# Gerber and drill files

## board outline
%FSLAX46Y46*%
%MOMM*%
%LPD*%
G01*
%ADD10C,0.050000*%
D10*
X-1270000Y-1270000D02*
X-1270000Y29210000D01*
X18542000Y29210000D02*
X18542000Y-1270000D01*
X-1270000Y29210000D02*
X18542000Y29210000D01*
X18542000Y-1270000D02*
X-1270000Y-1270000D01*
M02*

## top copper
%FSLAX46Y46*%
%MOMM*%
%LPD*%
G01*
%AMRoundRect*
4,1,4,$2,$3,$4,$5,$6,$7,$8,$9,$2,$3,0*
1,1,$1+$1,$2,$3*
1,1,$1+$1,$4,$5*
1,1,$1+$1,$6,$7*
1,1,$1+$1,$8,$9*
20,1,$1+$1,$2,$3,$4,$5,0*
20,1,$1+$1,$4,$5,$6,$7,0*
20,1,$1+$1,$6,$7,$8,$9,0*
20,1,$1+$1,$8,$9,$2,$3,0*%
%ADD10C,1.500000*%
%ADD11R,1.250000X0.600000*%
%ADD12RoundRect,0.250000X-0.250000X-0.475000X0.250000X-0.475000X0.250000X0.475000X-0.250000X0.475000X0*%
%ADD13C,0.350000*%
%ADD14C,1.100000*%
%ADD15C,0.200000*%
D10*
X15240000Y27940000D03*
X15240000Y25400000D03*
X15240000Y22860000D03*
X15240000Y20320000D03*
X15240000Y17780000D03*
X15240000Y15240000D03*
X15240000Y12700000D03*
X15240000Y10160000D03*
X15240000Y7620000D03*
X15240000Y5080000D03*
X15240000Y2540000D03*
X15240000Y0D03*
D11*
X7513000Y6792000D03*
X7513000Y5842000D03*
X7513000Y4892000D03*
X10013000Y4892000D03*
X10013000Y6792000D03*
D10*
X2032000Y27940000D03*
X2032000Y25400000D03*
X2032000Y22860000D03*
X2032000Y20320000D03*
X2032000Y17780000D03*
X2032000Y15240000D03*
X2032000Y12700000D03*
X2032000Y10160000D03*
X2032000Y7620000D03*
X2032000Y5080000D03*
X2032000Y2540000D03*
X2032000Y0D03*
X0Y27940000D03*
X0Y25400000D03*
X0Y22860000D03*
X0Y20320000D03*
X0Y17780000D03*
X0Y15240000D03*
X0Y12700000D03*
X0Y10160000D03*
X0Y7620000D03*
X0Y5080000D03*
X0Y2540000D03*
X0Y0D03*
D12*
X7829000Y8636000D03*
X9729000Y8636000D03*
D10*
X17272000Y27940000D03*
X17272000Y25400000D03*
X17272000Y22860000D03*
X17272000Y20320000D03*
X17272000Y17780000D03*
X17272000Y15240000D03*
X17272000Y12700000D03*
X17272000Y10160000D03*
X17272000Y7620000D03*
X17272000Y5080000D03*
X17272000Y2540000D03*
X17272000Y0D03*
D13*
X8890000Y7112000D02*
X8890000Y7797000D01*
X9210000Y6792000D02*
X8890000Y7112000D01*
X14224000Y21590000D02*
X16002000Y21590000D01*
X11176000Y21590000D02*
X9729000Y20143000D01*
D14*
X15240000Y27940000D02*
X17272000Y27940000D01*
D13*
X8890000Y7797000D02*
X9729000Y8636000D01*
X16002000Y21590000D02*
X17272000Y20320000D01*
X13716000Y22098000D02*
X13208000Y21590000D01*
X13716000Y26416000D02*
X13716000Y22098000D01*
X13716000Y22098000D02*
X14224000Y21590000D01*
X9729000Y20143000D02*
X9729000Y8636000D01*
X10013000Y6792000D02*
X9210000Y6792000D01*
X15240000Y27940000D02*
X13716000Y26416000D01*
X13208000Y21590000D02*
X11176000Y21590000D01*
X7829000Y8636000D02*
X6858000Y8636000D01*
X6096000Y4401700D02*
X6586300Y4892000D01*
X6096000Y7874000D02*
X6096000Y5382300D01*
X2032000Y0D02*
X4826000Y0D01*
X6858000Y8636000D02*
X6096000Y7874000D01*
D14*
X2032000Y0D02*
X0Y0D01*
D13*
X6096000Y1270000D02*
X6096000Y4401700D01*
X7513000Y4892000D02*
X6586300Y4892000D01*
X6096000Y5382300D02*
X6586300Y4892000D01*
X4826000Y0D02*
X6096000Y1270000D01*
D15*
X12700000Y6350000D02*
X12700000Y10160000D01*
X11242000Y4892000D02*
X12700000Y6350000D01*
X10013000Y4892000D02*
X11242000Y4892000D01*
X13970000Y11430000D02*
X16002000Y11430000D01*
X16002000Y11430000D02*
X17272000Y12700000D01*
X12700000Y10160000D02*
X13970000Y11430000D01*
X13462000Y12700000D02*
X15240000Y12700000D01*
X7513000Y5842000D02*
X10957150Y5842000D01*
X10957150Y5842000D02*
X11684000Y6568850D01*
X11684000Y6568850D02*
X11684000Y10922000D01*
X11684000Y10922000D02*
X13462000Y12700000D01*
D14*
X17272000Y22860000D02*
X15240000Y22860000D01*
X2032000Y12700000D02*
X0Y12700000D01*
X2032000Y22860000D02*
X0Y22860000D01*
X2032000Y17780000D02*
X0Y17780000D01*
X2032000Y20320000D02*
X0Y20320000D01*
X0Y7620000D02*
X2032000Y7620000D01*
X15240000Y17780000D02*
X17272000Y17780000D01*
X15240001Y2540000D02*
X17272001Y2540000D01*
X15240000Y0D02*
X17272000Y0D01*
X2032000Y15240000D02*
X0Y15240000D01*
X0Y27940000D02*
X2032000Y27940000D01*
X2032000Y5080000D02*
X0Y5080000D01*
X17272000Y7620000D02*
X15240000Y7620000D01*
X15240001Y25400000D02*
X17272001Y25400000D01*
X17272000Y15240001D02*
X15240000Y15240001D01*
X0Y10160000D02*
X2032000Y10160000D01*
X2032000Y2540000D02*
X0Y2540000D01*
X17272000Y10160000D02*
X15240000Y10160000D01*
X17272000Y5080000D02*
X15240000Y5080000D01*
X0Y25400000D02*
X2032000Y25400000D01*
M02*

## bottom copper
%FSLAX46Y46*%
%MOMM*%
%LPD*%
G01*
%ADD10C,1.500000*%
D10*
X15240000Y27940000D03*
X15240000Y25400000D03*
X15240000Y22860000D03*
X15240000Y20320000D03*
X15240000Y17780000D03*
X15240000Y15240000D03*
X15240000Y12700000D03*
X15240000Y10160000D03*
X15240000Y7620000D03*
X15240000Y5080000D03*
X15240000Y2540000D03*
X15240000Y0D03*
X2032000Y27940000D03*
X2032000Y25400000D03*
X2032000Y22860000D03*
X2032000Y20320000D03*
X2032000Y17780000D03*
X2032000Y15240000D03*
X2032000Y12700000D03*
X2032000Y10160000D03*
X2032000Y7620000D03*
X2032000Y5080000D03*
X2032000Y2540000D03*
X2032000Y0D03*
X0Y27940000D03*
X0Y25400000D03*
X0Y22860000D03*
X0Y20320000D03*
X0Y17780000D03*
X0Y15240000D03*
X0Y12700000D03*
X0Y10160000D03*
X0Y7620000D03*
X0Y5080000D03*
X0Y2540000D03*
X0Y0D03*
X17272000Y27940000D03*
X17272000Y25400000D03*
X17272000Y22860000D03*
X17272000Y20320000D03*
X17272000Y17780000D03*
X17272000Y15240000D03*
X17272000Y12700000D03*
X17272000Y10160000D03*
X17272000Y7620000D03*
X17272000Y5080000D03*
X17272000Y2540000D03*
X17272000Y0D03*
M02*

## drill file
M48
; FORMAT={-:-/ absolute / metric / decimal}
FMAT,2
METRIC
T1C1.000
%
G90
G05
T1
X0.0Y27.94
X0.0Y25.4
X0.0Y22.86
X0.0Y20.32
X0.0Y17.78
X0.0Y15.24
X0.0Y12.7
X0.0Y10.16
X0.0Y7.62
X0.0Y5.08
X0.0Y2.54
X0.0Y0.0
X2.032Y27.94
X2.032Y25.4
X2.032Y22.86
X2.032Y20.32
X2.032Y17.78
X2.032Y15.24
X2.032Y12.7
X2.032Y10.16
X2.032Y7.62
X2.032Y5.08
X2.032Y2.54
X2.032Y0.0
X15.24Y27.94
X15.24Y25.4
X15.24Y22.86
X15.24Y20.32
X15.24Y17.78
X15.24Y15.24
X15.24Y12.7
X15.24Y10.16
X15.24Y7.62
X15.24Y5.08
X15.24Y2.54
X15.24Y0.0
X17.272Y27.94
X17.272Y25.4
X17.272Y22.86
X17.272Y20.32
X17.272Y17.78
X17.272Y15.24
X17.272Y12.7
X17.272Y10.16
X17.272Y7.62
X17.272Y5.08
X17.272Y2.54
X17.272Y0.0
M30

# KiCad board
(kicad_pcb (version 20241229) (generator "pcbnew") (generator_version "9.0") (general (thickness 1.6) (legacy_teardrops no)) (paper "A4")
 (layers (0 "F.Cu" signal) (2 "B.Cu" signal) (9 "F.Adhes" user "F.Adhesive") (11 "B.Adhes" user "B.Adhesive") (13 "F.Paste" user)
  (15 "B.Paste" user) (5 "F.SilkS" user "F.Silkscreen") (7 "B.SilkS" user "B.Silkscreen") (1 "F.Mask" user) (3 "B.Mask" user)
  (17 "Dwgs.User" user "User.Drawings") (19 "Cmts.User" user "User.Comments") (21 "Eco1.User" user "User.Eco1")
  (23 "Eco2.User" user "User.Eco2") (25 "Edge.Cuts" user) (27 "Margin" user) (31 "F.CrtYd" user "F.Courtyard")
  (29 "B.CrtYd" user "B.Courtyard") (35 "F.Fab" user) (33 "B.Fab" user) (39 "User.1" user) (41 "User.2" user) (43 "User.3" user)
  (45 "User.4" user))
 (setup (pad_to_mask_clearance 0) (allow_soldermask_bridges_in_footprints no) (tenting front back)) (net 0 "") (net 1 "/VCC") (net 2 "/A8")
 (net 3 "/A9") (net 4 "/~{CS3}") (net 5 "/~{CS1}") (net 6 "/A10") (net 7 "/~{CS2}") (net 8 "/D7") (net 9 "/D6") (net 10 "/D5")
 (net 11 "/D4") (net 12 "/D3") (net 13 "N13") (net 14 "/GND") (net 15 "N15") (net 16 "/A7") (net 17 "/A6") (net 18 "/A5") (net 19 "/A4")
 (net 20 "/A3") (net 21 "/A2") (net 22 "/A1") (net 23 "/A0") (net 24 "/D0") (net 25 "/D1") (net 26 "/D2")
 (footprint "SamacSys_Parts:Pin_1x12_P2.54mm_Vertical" (layer "F.Cu") (at 15.24 -27.94)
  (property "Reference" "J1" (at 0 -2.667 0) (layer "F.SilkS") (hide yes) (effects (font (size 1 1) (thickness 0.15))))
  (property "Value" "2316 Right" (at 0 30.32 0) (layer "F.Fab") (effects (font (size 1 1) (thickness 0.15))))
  (pad "1" thru_hole circle (at 0 0) (size 1.5 1.5) (drill 1) (layers "*.Cu" "*.Mask") (remove_unused_layers no) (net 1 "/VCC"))
  (pad "2" thru_hole circle (at 0 2.54) (size 1.5 1.5) (drill 1) (layers "*.Cu" "*.Mask") (remove_unused_layers no) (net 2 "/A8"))
  (pad "3" thru_hole circle (at 0 5.08) (size 1.5 1.5) (drill 1) (layers "*.Cu" "*.Mask") (remove_unused_layers no) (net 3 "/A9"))
  (pad "4" thru_hole circle (at 0 7.62) (size 1.5 1.5) (drill 1) (layers "*.Cu" "*.Mask") (remove_unused_layers no) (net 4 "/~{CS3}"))
  (pad "5" thru_hole circle (at 0 10.16) (size 1.5 1.5) (drill 1) (layers "*.Cu" "*.Mask") (remove_unused_layers no) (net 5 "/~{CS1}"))
  (pad "6" thru_hole circle (at 0 12.7) (size 1.5 1.5) (drill 1) (layers "*.Cu" "*.Mask") (remove_unused_layers no) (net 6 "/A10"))
  (pad "7" thru_hole circle (at 0 15.24) (size 1.5 1.5) (drill 1) (layers "*.Cu" "*.Mask") (remove_unused_layers no) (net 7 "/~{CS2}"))
  (pad "8" thru_hole circle (at 0 17.78) (size 1.5 1.5) (drill 1) (layers "*.Cu" "*.Mask") (remove_unused_layers no) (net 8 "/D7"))
  (pad "9" thru_hole circle (at 0 20.32) (size 1.5 1.5) (drill 1) (layers "*.Cu" "*.Mask") (remove_unused_layers no) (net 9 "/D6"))
  (pad "10" thru_hole circle (at 0 22.86) (size 1.5 1.5) (drill 1) (layers "*.Cu" "*.Mask") (remove_unused_layers no) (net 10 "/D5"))
  (pad "11" thru_hole circle (at 0 25.4) (size 1.5 1.5) (drill 1) (layers "*.Cu" "*.Mask") (remove_unused_layers no) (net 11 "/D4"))
  (pad "12" thru_hole circle (at 0 27.94) (size 1.5 1.5) (drill 1) (layers "*.Cu" "*.Mask") (remove_unused_layers no) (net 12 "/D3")))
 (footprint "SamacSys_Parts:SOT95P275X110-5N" (layer "F.Cu") (at 8.763 -5.842)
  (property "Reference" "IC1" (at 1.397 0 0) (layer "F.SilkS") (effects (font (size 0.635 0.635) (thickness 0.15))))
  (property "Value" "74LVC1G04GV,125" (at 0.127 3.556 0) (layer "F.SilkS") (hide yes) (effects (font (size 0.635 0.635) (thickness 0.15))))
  (pad "1" smd rect (at -1.25 -0.95 90) (size 0.6 1.25) (layers "F.Cu" "F.Mask" "F.Paste") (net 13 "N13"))
  (pad "2" smd rect (at -1.25 0 90) (size 0.6 1.25) (layers "F.Cu" "F.Mask" "F.Paste") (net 7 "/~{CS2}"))
  (pad "3" smd rect (at -1.25 0.95 90) (size 0.6 1.25) (layers "F.Cu" "F.Mask" "F.Paste") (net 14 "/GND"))
  (pad "4" smd rect (at 1.25 0.95 90) (size 0.6 1.25) (layers "F.Cu" "F.Mask" "F.Paste") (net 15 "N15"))
  (pad "5" smd rect (at 1.25 -0.95 90) (size 0.6 1.25) (layers "F.Cu" "F.Mask" "F.Paste") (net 1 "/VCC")))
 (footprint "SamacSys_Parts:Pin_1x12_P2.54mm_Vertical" (layer "F.Cu") (at 2.032 -27.94)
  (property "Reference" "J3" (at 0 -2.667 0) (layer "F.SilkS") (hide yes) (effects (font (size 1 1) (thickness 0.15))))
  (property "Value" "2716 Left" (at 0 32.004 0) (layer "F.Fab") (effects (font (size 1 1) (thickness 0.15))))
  (pad "1" thru_hole circle (at 0 0) (size 1.5 1.5) (drill 1) (layers "*.Cu" "*.Mask") (remove_unused_layers no) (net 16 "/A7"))
  (pad "2" thru_hole circle (at 0 2.54) (size 1.5 1.5) (drill 1) (layers "*.Cu" "*.Mask") (remove_unused_layers no) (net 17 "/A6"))
  (pad "3" thru_hole circle (at 0 5.08) (size 1.5 1.5) (drill 1) (layers "*.Cu" "*.Mask") (remove_unused_layers no) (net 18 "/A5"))
  (pad "4" thru_hole circle (at 0 7.62) (size 1.5 1.5) (drill 1) (layers "*.Cu" "*.Mask") (remove_unused_layers no) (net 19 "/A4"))
  (pad "5" thru_hole circle (at 0 10.16) (size 1.5 1.5) (drill 1) (layers "*.Cu" "*.Mask") (remove_unused_layers no) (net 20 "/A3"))
  (pad "6" thru_hole circle (at 0 12.7) (size 1.5 1.5) (drill 1) (layers "*.Cu" "*.Mask") (remove_unused_layers no) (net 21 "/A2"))
  (pad "7" thru_hole circle (at 0 15.24) (size 1.5 1.5) (drill 1) (layers "*.Cu" "*.Mask") (remove_unused_layers no) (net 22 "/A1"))
  (pad "8" thru_hole circle (at 0 17.78) (size 1.5 1.5) (drill 1) (layers "*.Cu" "*.Mask") (remove_unused_layers no) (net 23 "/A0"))
  (pad "9" thru_hole circle (at 0 20.32) (size 1.5 1.5) (drill 1) (layers "*.Cu" "*.Mask") (remove_unused_layers no) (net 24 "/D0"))
  (pad "10" thru_hole circle (at 0 22.86) (size 1.5 1.5) (drill 1) (layers "*.Cu" "*.Mask") (remove_unused_layers no) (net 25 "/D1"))
  (pad "11" thru_hole circle (at 0 25.4) (size 1.5 1.5) (drill 1) (layers "*.Cu" "*.Mask") (remove_unused_layers no) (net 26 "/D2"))
  (pad "12" thru_hole circle (at 0 27.94) (size 1.5 1.5) (drill 1) (layers "*.Cu" "*.Mask") (remove_unused_layers no) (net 14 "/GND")))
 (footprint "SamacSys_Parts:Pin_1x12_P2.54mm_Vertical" (layer "F.Cu") (at 0 -27.94)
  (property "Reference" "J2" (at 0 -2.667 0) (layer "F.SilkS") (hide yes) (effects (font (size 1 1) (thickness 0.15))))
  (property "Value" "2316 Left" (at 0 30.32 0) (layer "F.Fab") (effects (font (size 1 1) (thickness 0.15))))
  (pad "1" thru_hole circle (at 0 0) (size 1.5 1.5) (drill 1) (layers "*.Cu" "*.Mask") (remove_unused_layers no) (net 16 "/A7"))
  (pad "2" thru_hole circle (at 0 2.54) (size 1.5 1.5) (drill 1) (layers "*.Cu" "*.Mask") (remove_unused_layers no) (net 17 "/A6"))
  (pad "3" thru_hole circle (at 0 5.08) (size 1.5 1.5) (drill 1) (layers "*.Cu" "*.Mask") (remove_unused_layers no) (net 18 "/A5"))
  (pad "4" thru_hole circle (at 0 7.62) (size 1.5 1.5) (drill 1) (layers "*.Cu" "*.Mask") (remove_unused_layers no) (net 19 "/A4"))
  (pad "5" thru_hole circle (at 0 10.16) (size 1.5 1.5) (drill 1) (layers "*.Cu" "*.Mask") (remove_unused_layers no) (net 20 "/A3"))
  (pad "6" thru_hole circle (at 0 12.7) (size 1.5 1.5) (drill 1) (layers "*.Cu" "*.Mask") (remove_unused_layers no) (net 21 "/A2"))
  (pad "7" thru_hole circle (at 0 15.24) (size 1.5 1.5) (drill 1) (layers "*.Cu" "*.Mask") (remove_unused_layers no) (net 22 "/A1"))
  (pad "8" thru_hole circle (at 0 17.78) (size 1.5 1.5) (drill 1) (layers "*.Cu" "*.Mask") (remove_unused_layers no) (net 23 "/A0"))
  (pad "9" thru_hole circle (at 0 20.32) (size 1.5 1.5) (drill 1) (layers "*.Cu" "*.Mask") (remove_unused_layers no) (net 24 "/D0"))
  (pad "10" thru_hole circle (at 0 22.86) (size 1.5 1.5) (drill 1) (layers "*.Cu" "*.Mask") (remove_unused_layers no) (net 25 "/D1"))
  (pad "11" thru_hole circle (at 0 25.4) (size 1.5 1.5) (drill 1) (layers "*.Cu" "*.Mask") (remove_unused_layers no) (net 26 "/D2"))
  (pad "12" thru_hole circle (at 0 27.94) (size 1.5 1.5) (drill 1) (layers "*.Cu" "*.Mask") (remove_unused_layers no) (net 14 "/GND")))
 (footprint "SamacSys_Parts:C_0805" (layer "F.Cu") (at 8.763 -8.636 -90)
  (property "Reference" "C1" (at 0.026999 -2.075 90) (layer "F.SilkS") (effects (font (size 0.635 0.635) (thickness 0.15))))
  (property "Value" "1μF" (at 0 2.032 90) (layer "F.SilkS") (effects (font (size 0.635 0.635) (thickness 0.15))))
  (pad "1" smd roundrect (at 0 0.934) (size 1 1.45) (layers "F.Cu" "F.Mask" "F.Paste") (roundrect_rratio 0.25) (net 14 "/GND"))
  (pad "2" smd roundrect (at 0 -0.966) (size 1 1.45) (layers "F.Cu" "F.Mask" "F.Paste") (roundrect_rratio 0.25) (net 1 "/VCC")))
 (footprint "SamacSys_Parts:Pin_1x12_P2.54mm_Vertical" (layer "F.Cu") (at 17.272 -27.94)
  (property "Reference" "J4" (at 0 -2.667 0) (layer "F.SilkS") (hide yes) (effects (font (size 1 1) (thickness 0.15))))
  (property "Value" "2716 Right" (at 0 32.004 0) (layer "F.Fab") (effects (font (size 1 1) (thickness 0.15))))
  (pad "1" thru_hole circle (at 0 0) (size 1.5 1.5) (drill 1) (layers "*.Cu" "*.Mask") (remove_unused_layers no) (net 1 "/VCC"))
  (pad "2" thru_hole circle (at 0 2.54) (size 1.5 1.5) (drill 1) (layers "*.Cu" "*.Mask") (remove_unused_layers no) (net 2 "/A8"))
  (pad "3" thru_hole circle (at 0 5.08) (size 1.5 1.5) (drill 1) (layers "*.Cu" "*.Mask") (remove_unused_layers no) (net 3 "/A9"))
  (pad "4" thru_hole circle (at 0 7.62) (size 1.5 1.5) (drill 1) (layers "*.Cu" "*.Mask") (remove_unused_layers no) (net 1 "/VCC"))
  (pad "5" thru_hole circle (at 0 10.16) (size 1.5 1.5) (drill 1) (layers "*.Cu" "*.Mask") (remove_unused_layers no) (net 5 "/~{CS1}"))
  (pad "6" thru_hole circle (at 0 12.7) (size 1.5 1.5) (drill 1) (layers "*.Cu" "*.Mask") (remove_unused_layers no) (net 6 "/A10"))
  (pad "7" thru_hole circle (at 0 15.24) (size 1.5 1.5) (drill 1) (layers "*.Cu" "*.Mask") (remove_unused_layers no) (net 15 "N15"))
  (pad "8" thru_hole circle (at 0 17.78) (size 1.5 1.5) (drill 1) (layers "*.Cu" "*.Mask") (remove_unused_layers no) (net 8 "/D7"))
  (pad "9" thru_hole circle (at 0 20.32) (size 1.5 1.5) (drill 1) (layers "*.Cu" "*.Mask") (remove_unused_layers no) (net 9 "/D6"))
  (pad "10" thru_hole circle (at 0 22.86) (size 1.5 1.5) (drill 1) (layers "*.Cu" "*.Mask") (remove_unused_layers no) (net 10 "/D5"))
  (pad "11" thru_hole circle (at 0 25.4) (size 1.5 1.5) (drill 1) (layers "*.Cu" "*.Mask") (remove_unused_layers no) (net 11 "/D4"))
  (pad "12" thru_hole circle (at 0 27.94) (size 1.5 1.5) (drill 1) (layers "*.Cu" "*.Mask") (remove_unused_layers no) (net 12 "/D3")))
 (gr_line (start -1.27 1.27) (end -1.27 -29.21) (stroke (width 0.05) (type default)) (layer "Edge.Cuts"))
 (gr_line (start 18.542 -29.21) (end 18.542 1.27) (stroke (width 0.05) (type default)) (layer "Edge.Cuts"))
 (gr_line (start -1.27 -29.21) (end 18.542 -29.21) (stroke (width 0.05) (type default)) (layer "Edge.Cuts"))
 (gr_line (start 18.542 1.27) (end -1.27 1.27) (stroke (width 0.05) (type default)) (layer "Edge.Cuts"))
 (segment (start 8.89 -7.112) (end 8.89 -7.797) (width 0.35) (layer "F.Cu") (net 1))
 (segment (start 9.21 -6.792) (end 8.89 -7.112) (width 0.35) (layer "F.Cu") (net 1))
 (segment (start 14.224 -21.59) (end 16.002 -21.59) (width 0.35) (layer "F.Cu") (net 1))
 (segment (start 11.176 -21.59) (end 9.729 -20.143) (width 0.35) (layer "F.Cu") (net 1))
 (segment (start 15.24 -27.94) (end 17.272 -27.94) (width 1.1) (layer "F.Cu") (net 1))
 (segment (start 8.89 -7.797) (end 9.729 -8.636) (width 0.35) (layer "F.Cu") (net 1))
 (segment (start 16.002 -21.59) (end 17.272 -20.32) (width 0.35) (layer "F.Cu") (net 1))
 (segment (start 13.716 -22.098) (end 13.208 -21.59) (width 0.35) (layer "F.Cu") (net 1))
 (segment (start 13.716 -26.416) (end 13.716 -22.098) (width 0.35) (layer "F.Cu") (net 1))
 (segment (start 13.716 -22.098) (end 14.224 -21.59) (width 0.35) (layer "F.Cu") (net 1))
 (segment (start 9.729 -20.143) (end 9.729 -8.636) (width 0.35) (layer "F.Cu") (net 1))
 (segment (start 10.013 -6.792) (end 9.21 -6.792) (width 0.35) (layer "F.Cu") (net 1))
 (segment (start 15.24 -27.94) (end 13.716 -26.416) (width 0.35) (layer "F.Cu") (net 1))
 (segment (start 13.208 -21.59) (end 11.176 -21.59) (width 0.35) (layer "F.Cu") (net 1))
 (segment (start 7.829 -8.636) (end 6.858 -8.636) (width 0.35) (layer "F.Cu") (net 14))
 (segment (start 6.096 -4.4017) (end 6.5863 -4.892) (width 0.35) (layer "F.Cu") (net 14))
 (segment (start 6.096 -7.874) (end 6.096 -5.3823) (width 0.35) (layer "F.Cu") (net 14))
 (segment (start 2.032 0) (end 4.826 0) (width 0.35) (layer "F.Cu") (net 14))
 (segment (start 6.858 -8.636) (end 6.096 -7.874) (width 0.35) (layer "F.Cu") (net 14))
 (segment (start 2.032 0) (end 0 0) (width 1.1) (layer "F.Cu") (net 14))
 (segment (start 6.096 -1.27) (end 6.096 -4.4017) (width 0.35) (layer "F.Cu") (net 14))
 (segment (start 7.513 -4.892) (end 6.5863 -4.892) (width 0.35) (layer "F.Cu") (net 14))
 (segment (start 6.096 -5.3823) (end 6.5863 -4.892) (width 0.35) (layer "F.Cu") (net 14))
 (segment (start 4.826 0) (end 6.096 -1.27) (width 0.35) (layer "F.Cu") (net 14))
 (segment (start 12.7 -6.35) (end 12.7 -10.16) (width 0.2) (layer "F.Cu") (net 15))
 (segment (start 11.242 -4.892) (end 12.7 -6.35) (width 0.2) (layer "F.Cu") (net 15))
 (segment (start 10.013 -4.892) (end 11.242 -4.892) (width 0.2) (layer "F.Cu") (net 15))
 (segment (start 13.97 -11.43) (end 16.002 -11.43) (width 0.2) (layer "F.Cu") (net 15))
 (segment (start 16.002 -11.43) (end 17.272 -12.7) (width 0.2) (layer "F.Cu") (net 15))
 (segment (start 12.7 -10.16) (end 13.97 -11.43) (width 0.2) (layer "F.Cu") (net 15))
 (segment (start 13.462 -12.7) (end 15.24 -12.7) (width 0.2) (layer "F.Cu") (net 7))
 (segment (start 7.513 -5.842) (end 10.95715 -5.842) (width 0.2) (layer "F.Cu") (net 7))
 (segment (start 10.95715 -5.842) (end 11.684 -6.56885) (width 0.2) (layer "F.Cu") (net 7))
 (segment (start 11.684 -6.56885) (end 11.684 -10.922) (width 0.2) (layer "F.Cu") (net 7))
 (segment (start 11.684 -10.922) (end 13.462 -12.7) (width 0.2) (layer "F.Cu") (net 7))
 (segment (start 17.272 -22.86) (end 15.24 -22.86) (width 1.1) (layer "F.Cu") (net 3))
 (segment (start 2.032 -12.7) (end 0 -12.7) (width 1.1) (layer "F.Cu") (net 22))
 (segment (start 2.032 -22.86) (end 0 -22.86) (width 1.1) (layer "F.Cu") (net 18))
 (segment (start 2.032 -17.78) (end 0 -17.78) (width 1.1) (layer "F.Cu") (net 20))
 (segment (start 2.032 -20.32) (end 0 -20.32) (width 1.1) (layer "F.Cu") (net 19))
 (segment (start 0 -7.62) (end 2.032 -7.62) (width 1.1) (layer "F.Cu") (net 24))
 (segment (start 15.24 -17.78) (end 17.272 -17.78) (width 1.1) (layer "F.Cu") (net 5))
 (segment (start 15.240001 -2.54) (end 17.272001 -2.54) (width 1.1) (layer "F.Cu") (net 11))
 (segment (start 15.24 0) (end 17.272 0) (width 1.1) (layer "F.Cu") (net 12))
 (segment (start 2.032 -15.24) (end 0 -15.24) (width 1.1) (layer "F.Cu") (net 21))
 (segment (start 0 -27.94) (end 2.032 -27.94) (width 1.1) (layer "F.Cu") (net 16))
 (segment (start 2.032 -5.08) (end 0 -5.08) (width 1.1) (layer "F.Cu") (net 25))
 (segment (start 17.272 -7.62) (end 15.24 -7.62) (width 1.1) (layer "F.Cu") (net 9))
 (segment (start 15.240001 -25.4) (end 17.272001 -25.4) (width 1.1) (layer "F.Cu") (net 2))
 (segment (start 17.272 -15.240001) (end 15.24 -15.240001) (width 1.1) (layer "F.Cu") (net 6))
 (segment (start 0 -10.16) (end 2.032 -10.16) (width 1.1) (layer "F.Cu") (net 23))
 (segment (start 2.032 -2.54) (end 0 -2.54) (width 1.1) (layer "F.Cu") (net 26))
 (segment (start 17.272 -10.16) (end 15.24 -10.16) (width 1.1) (layer "F.Cu") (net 8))
 (segment (start 17.272 -5.08) (end 15.24 -5.08) (width 1.1) (layer "F.Cu") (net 10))
 (segment (start 0 -25.4) (end 2.032 -25.4) (width 1.1) (layer "F.Cu") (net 17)))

